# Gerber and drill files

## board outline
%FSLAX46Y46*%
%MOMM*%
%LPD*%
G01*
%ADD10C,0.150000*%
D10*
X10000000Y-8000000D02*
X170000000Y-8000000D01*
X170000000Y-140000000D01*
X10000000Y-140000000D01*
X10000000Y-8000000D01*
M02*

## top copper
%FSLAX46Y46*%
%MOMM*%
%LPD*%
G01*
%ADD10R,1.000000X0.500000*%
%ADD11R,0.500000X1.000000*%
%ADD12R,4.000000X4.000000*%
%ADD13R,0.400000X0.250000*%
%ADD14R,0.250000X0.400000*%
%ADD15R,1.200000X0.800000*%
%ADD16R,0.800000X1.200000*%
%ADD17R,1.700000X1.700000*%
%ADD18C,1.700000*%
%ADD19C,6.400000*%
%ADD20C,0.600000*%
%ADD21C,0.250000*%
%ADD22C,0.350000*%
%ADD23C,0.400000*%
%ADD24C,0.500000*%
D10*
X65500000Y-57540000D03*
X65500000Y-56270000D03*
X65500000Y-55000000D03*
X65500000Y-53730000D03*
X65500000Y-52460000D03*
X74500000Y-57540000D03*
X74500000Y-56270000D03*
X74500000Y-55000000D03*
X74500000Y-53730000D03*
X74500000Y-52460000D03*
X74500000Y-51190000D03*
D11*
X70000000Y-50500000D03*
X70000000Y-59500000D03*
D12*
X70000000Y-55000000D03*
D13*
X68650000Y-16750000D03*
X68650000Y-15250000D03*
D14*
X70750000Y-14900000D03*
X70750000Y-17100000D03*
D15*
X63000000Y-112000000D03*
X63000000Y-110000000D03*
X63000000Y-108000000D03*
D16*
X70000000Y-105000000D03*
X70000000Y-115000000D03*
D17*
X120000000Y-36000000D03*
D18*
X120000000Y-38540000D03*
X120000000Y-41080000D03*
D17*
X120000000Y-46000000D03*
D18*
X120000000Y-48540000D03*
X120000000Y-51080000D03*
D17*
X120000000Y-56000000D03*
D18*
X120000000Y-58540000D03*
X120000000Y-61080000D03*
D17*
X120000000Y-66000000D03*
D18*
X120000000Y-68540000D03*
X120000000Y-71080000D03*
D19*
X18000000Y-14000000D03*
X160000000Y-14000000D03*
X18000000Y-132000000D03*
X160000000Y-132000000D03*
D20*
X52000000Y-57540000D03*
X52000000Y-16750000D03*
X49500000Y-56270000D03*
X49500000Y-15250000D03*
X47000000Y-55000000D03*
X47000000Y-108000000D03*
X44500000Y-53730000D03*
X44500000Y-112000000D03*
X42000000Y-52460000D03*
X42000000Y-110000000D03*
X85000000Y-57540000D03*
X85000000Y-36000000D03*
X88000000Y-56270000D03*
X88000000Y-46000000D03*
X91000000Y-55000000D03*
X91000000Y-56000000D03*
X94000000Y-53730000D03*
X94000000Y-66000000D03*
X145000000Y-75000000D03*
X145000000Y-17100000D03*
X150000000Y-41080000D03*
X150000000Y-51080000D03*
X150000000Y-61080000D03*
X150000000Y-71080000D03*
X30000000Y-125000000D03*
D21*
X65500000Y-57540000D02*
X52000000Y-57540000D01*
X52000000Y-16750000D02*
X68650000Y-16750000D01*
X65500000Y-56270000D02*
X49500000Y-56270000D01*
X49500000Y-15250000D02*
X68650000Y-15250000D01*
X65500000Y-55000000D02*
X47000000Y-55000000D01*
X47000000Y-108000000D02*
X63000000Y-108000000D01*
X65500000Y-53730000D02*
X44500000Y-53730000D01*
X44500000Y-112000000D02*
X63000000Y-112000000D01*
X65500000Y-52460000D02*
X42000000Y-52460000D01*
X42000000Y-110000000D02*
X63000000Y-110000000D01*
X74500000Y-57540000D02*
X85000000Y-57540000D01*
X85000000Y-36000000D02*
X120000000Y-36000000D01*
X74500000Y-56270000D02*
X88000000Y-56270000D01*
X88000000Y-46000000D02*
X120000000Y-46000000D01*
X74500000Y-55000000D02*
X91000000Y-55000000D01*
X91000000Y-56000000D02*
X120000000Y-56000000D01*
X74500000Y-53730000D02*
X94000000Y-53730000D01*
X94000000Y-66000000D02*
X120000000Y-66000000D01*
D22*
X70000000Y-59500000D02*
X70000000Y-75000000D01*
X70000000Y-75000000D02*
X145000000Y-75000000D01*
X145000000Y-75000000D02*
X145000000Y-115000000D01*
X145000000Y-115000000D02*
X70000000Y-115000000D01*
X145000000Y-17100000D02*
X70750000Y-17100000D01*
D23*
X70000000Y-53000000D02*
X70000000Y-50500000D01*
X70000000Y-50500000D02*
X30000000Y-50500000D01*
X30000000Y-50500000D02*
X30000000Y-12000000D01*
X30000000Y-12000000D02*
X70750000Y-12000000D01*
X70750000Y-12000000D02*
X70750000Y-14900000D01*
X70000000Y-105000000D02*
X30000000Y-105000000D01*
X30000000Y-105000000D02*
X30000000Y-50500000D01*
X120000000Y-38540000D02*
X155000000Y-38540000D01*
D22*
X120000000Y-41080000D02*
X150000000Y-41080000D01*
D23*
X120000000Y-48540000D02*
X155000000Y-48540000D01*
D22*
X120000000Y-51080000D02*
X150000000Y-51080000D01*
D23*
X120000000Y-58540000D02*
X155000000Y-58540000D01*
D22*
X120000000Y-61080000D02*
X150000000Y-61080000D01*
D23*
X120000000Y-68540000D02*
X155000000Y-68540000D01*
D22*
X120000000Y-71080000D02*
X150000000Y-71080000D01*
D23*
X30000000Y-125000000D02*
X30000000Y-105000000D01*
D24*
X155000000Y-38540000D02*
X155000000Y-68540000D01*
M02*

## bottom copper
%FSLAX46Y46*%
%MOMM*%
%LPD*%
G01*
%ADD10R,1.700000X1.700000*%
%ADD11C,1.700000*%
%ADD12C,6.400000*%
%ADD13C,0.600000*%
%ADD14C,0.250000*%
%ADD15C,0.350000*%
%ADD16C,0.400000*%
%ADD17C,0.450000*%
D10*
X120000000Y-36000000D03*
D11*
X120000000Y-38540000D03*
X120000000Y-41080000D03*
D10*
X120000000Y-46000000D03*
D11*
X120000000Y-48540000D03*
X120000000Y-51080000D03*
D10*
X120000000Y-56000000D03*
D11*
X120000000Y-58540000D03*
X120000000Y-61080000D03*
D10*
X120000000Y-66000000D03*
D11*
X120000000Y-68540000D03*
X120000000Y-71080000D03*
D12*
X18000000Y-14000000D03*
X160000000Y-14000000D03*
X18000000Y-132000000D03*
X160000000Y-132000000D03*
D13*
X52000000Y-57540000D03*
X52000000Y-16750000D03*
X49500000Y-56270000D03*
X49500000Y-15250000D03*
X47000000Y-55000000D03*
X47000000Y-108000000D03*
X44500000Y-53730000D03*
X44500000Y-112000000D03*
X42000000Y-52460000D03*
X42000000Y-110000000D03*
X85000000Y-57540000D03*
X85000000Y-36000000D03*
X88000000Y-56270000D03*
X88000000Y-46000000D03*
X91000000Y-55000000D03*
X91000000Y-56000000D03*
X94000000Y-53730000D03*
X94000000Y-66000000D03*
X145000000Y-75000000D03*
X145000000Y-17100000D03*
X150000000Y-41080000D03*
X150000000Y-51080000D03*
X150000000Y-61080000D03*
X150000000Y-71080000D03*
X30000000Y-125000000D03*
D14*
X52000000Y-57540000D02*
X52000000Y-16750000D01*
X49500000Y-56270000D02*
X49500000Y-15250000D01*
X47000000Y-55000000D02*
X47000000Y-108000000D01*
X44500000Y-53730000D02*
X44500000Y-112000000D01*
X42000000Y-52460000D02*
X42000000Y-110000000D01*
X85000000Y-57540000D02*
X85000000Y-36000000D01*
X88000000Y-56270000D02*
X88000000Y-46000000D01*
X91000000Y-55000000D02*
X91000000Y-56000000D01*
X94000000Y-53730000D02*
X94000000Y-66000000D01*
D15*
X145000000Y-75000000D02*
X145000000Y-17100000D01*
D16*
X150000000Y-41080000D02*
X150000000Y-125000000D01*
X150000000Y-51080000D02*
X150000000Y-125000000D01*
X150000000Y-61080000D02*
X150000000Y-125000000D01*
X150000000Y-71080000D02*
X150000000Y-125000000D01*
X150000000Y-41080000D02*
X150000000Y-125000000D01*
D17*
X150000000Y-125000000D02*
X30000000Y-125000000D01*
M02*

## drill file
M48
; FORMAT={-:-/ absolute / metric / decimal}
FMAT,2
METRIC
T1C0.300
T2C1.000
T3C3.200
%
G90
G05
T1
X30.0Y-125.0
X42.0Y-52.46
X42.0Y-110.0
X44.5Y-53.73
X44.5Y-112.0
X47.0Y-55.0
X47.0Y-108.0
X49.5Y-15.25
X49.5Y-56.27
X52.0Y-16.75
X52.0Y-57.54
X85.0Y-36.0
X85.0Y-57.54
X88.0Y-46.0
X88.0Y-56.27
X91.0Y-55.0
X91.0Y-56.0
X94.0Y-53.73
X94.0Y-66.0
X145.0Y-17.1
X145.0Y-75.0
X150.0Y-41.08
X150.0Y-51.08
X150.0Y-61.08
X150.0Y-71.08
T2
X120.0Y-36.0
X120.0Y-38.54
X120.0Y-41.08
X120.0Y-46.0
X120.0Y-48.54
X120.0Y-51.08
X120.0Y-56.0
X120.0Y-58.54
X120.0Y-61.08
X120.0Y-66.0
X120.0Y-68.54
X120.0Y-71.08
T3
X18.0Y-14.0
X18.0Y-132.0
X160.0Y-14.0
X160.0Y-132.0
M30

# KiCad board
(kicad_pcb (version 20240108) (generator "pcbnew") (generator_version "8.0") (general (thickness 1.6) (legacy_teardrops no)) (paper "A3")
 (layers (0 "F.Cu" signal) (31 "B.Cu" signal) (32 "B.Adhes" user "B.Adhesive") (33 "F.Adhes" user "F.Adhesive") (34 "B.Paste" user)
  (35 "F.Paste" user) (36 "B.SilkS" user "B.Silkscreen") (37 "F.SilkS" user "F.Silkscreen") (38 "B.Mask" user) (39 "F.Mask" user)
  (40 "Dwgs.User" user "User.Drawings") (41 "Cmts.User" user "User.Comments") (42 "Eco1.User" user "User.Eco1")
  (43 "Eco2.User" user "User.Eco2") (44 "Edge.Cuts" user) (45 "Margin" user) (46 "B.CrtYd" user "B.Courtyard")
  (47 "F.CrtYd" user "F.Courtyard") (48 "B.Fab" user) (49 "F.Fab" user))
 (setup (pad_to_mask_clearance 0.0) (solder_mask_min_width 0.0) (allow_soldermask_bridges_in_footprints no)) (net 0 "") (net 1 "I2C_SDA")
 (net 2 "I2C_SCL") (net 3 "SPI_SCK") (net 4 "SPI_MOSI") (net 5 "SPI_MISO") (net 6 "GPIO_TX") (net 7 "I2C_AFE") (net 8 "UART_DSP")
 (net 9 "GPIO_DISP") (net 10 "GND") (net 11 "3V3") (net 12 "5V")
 (gr_rect (start 10 8) (end 170 140) (stroke (width 0.15) (type solid)) (fill none) (layer "Edge.Cuts"))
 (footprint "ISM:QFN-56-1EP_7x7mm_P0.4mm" (layer "F.Cu") (at 70 55)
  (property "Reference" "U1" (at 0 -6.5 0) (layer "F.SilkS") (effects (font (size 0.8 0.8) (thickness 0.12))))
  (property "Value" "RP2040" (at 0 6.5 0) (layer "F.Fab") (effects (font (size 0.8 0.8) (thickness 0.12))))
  (pad "1" smd rect (at -4.5 2.54) (size 1.0 0.5) (layers "F.Cu" "F.Paste" "F.Mask") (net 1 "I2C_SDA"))
  (pad "2" smd rect (at -4.5 1.27) (size 1.0 0.5) (layers "F.Cu" "F.Paste" "F.Mask") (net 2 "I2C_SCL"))
  (pad "3" smd rect (at -4.5 0) (size 1.0 0.5) (layers "F.Cu" "F.Paste" "F.Mask") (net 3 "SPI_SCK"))
  (pad "4" smd rect (at -4.5 -1.27) (size 1.0 0.5) (layers "F.Cu" "F.Paste" "F.Mask") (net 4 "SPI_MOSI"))
  (pad "5" smd rect (at -4.5 -2.54) (size 1.0 0.5) (layers "F.Cu" "F.Paste" "F.Mask") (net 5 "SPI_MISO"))
  (pad "6" smd rect (at 4.5 2.54) (size 1.0 0.5) (layers "F.Cu" "F.Paste" "F.Mask") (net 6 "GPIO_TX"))
  (pad "7" smd rect (at 4.5 1.27) (size 1.0 0.5) (layers "F.Cu" "F.Paste" "F.Mask") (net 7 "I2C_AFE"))
  (pad "8" smd rect (at 4.5 0) (size 1.0 0.5) (layers "F.Cu" "F.Paste" "F.Mask") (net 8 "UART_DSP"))
  (pad "9" smd rect (at 4.5 -1.27) (size 1.0 0.5) (layers "F.Cu" "F.Paste" "F.Mask") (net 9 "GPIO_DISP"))
  (pad "12" smd rect (at 4.5 -2.54) (size 1.0 0.5) (layers "F.Cu" "F.Paste" "F.Mask"))
  (pad "13" smd rect (at 4.5 -3.81) (size 1.0 0.5) (layers "F.Cu" "F.Paste" "F.Mask"))
  (pad "10" smd rect (at 0 -4.5) (size 0.5 1.0) (layers "F.Cu" "F.Paste" "F.Mask") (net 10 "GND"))
  (pad "11" smd rect (at 0 4.5) (size 0.5 1.0) (layers "F.Cu" "F.Paste" "F.Mask") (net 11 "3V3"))
  (pad "EP" smd rect (at 0 0) (size 4 4) (layers "F.Cu" "F.Paste" "F.Mask") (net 10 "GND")))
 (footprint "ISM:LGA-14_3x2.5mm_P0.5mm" (layer "F.Cu") (at 70 16)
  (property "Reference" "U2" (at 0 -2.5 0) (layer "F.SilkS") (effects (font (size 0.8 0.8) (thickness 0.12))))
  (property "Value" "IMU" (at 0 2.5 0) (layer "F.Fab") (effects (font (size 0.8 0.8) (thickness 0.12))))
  (pad "1" smd rect (at -1.35 0.75) (size 0.4 0.25) (layers "F.Cu" "F.Paste" "F.Mask") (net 1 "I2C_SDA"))
  (pad "2" smd rect (at -1.35 -0.75) (size 0.4 0.25) (layers "F.Cu" "F.Paste" "F.Mask") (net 2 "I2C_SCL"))
  (pad "3" smd rect (at 0.75 -1.1) (size 0.25 0.4) (layers "F.Cu" "F.Paste" "F.Mask") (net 10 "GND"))
  (pad "4" smd rect (at 0.75 1.1) (size 0.25 0.4) (layers "F.Cu" "F.Paste" "F.Mask") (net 11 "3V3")))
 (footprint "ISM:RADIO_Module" (layer "F.Cu") (at 70 110)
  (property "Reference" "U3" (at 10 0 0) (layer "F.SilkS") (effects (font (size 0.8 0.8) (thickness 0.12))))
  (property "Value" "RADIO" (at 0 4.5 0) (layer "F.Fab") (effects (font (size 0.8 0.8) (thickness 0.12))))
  (pad "1" smd rect (at -7 2) (size 1.2 0.8) (layers "F.Cu" "F.Paste" "F.Mask") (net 4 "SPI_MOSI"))
  (pad "2" smd rect (at -7 0) (size 1.2 0.8) (layers "F.Cu" "F.Paste" "F.Mask") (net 5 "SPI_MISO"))
  (pad "3" smd rect (at -7 -2) (size 1.2 0.8) (layers "F.Cu" "F.Paste" "F.Mask") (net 3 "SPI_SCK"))
  (pad "4" smd rect (at 0 -5) (size 0.8 1.2) (layers "F.Cu" "F.Paste" "F.Mask") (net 10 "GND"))
  (pad "5" smd rect (at 0 5) (size 0.8 1.2) (layers "F.Cu" "F.Paste" "F.Mask") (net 11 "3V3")))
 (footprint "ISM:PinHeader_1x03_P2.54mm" (layer "F.Cu") (at 120 36)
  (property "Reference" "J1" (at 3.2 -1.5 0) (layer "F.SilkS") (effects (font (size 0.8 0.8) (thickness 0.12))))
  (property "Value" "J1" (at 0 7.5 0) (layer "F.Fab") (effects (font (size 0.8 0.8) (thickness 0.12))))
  (pad "1" thru_hole rect (at 0 0) (size 1.7 1.7) (drill 1.0) (layers "*.Cu" "*.Mask") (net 6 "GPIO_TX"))
  (pad "2" thru_hole circle (at 0 2.54) (size 1.7 1.7) (drill 1.0) (layers "*.Cu" "*.Mask") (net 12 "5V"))
  (pad "3" thru_hole circle (at 0 5.08) (size 1.7 1.7) (drill 1.0) (layers "*.Cu" "*.Mask") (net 10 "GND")))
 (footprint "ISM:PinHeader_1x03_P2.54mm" (layer "F.Cu") (at 120 46)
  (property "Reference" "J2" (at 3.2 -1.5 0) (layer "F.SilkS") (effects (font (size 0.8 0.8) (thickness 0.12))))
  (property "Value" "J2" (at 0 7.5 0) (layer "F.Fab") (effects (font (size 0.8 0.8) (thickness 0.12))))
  (pad "1" thru_hole rect (at 0 0) (size 1.7 1.7) (drill 1.0) (layers "*.Cu" "*.Mask") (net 7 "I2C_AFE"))
  (pad "2" thru_hole circle (at 0 2.54) (size 1.7 1.7) (drill 1.0) (layers "*.Cu" "*.Mask") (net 12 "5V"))
  (pad "3" thru_hole circle (at 0 5.08) (size 1.7 1.7) (drill 1.0) (layers "*.Cu" "*.Mask") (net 10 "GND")))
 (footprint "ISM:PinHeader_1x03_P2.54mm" (layer "F.Cu") (at 120 56)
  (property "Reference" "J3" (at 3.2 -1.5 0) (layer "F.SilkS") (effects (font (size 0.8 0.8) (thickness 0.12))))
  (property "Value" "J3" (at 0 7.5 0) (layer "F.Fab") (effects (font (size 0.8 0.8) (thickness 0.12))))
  (pad "1" thru_hole rect (at 0 0) (size 1.7 1.7) (drill 1.0) (layers "*.Cu" "*.Mask") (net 8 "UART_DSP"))
  (pad "2" thru_hole circle (at 0 2.54) (size 1.7 1.7) (drill 1.0) (layers "*.Cu" "*.Mask") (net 12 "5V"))
  (pad "3" thru_hole circle (at 0 5.08) (size 1.7 1.7) (drill 1.0) (layers "*.Cu" "*.Mask") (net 10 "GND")))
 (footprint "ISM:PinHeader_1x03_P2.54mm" (layer "F.Cu") (at 120 66)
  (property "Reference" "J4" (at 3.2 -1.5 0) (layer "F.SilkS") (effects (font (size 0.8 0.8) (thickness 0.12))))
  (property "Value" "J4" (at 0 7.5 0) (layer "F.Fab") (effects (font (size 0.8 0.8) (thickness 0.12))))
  (pad "1" thru_hole rect (at 0 0) (size 1.7 1.7) (drill 1.0) (layers "*.Cu" "*.Mask") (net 9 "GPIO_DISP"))
  (pad "2" thru_hole circle (at 0 2.54) (size 1.7 1.7) (drill 1.0) (layers "*.Cu" "*.Mask") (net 12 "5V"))
  (pad "3" thru_hole circle (at 0 5.08) (size 1.7 1.7) (drill 1.0) (layers "*.Cu" "*.Mask") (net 10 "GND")))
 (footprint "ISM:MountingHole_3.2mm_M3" (layer "F.Cu") (at 18 14)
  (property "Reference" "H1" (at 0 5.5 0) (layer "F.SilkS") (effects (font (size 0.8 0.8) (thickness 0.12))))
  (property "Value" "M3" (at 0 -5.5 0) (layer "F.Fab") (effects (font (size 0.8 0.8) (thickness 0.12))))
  (pad "" thru_hole circle (at 0 0) (size 6.4 6.4) (drill 3.2) (layers "*.Cu" "*.Mask")))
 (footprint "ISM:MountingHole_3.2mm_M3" (layer "F.Cu") (at 160 14)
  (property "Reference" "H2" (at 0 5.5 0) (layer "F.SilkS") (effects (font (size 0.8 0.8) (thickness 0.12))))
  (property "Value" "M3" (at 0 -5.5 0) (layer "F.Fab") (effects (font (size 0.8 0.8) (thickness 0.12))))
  (pad "" thru_hole circle (at 0 0) (size 6.4 6.4) (drill 3.2) (layers "*.Cu" "*.Mask")))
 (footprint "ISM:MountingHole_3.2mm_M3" (layer "F.Cu") (at 18 132)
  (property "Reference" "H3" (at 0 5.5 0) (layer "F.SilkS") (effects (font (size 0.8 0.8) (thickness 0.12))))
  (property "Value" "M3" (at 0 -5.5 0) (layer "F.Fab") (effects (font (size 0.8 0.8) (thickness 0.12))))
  (pad "" thru_hole circle (at 0 0) (size 6.4 6.4) (drill 3.2) (layers "*.Cu" "*.Mask")))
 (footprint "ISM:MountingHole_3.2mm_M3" (layer "F.Cu") (at 160 132)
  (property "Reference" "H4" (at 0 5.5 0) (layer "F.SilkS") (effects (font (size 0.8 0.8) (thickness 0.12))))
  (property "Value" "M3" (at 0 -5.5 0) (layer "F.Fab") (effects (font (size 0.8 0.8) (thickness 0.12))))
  (pad "" thru_hole circle (at 0 0) (size 6.4 6.4) (drill 3.2) (layers "*.Cu" "*.Mask")))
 (segment (start 65.5 57.54) (end 52.0 57.54) (width 0.25) (layer "F.Cu") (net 1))
 (segment (start 52.0 57.54) (end 52.0 16.75) (width 0.25) (layer "B.Cu") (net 1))
 (segment (start 52.0 16.75) (end 68.65 16.75) (width 0.25) (layer "F.Cu") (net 1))
 (segment (start 65.5 56.27) (end 49.5 56.27) (width 0.25) (layer "F.Cu") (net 2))
 (segment (start 49.5 56.27) (end 49.5 15.25) (width 0.25) (layer "B.Cu") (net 2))
 (segment (start 49.5 15.25) (end 68.65 15.25) (width 0.25) (layer "F.Cu") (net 2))
 (segment (start 65.5 55) (end 47.0 55) (width 0.25) (layer "F.Cu") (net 3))
 (segment (start 47.0 55) (end 47.0 108) (width 0.25) (layer "B.Cu") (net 3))
 (segment (start 47.0 108) (end 63 108) (width 0.25) (layer "F.Cu") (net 3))
 (segment (start 65.5 53.73) (end 44.5 53.73) (width 0.25) (layer "F.Cu") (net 4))
 (segment (start 44.5 53.73) (end 44.5 112) (width 0.25) (layer "B.Cu") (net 4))
 (segment (start 44.5 112) (end 63 112) (width 0.25) (layer "F.Cu") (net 4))
 (segment (start 65.5 52.46) (end 42.0 52.46) (width 0.25) (layer "F.Cu") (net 5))
 (segment (start 42.0 52.46) (end 42.0 110) (width 0.25) (layer "B.Cu") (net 5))
 (segment (start 42.0 110) (end 63 110) (width 0.25) (layer "F.Cu") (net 5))
 (segment (start 74.5 57.54) (end 85 57.54) (width 0.25) (layer "F.Cu") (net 6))
 (segment (start 85 57.54) (end 85 36) (width 0.25) (layer "B.Cu") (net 6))
 (segment (start 85 36) (end 120 36) (width 0.25) (layer "F.Cu") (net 6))
 (segment (start 74.5 56.27) (end 88 56.27) (width 0.25) (layer "F.Cu") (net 7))
 (segment (start 88 56.27) (end 88 46) (width 0.25) (layer "B.Cu") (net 7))
 (segment (start 88 46) (end 120 46) (width 0.25) (layer "F.Cu") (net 7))
 (segment (start 74.5 55) (end 91 55) (width 0.25) (layer "F.Cu") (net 8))
 (segment (start 91 55) (end 91 56) (width 0.25) (layer "B.Cu") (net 8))
 (segment (start 91 56) (end 120 56) (width 0.25) (layer "F.Cu") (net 8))
 (segment (start 74.5 53.73) (end 94 53.73) (width 0.25) (layer "F.Cu") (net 9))
 (segment (start 94 53.73) (end 94 66) (width 0.25) (layer "B.Cu") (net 9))
 (segment (start 94 66) (end 120 66) (width 0.25) (layer "F.Cu") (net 9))
 (segment (start 70 59.5) (end 70 75) (width 0.35) (layer "F.Cu") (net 11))
 (segment (start 70 75) (end 145 75) (width 0.35) (layer "F.Cu") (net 11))
 (segment (start 145 75) (end 145 115) (width 0.35) (layer "F.Cu") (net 11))
 (segment (start 145 115) (end 70 115) (width 0.35) (layer "F.Cu") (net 11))
 (segment (start 145 75) (end 145 17.1) (width 0.35) (layer "B.Cu") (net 11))
 (segment (start 145 17.1) (end 70.75 17.1) (width 0.35) (layer "F.Cu") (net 11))
 (segment (start 70 53) (end 70 50.5) (width 0.4) (layer "F.Cu") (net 10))
 (segment (start 70 50.5) (end 30 50.5) (width 0.4) (layer "F.Cu") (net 10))
 (segment (start 30 50.5) (end 30 12) (width 0.4) (layer "F.Cu") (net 10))
 (segment (start 30 12) (end 70.75 12) (width 0.4) (layer "F.Cu") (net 10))
 (segment (start 70.75 12) (end 70.75 14.9) (width 0.4) (layer "F.Cu") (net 10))
 (segment (start 70 105) (end 30 105) (width 0.4) (layer "F.Cu") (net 10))
 (segment (start 30 105) (end 30 50.5) (width 0.4) (layer "F.Cu") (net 10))
 (segment (start 120 38.54) (end 155 38.54) (width 0.4) (layer "F.Cu") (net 12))
 (segment (start 120 41.08) (end 150 41.08) (width 0.35) (layer "F.Cu") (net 10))
 (segment (start 150 41.08) (end 150 125) (width 0.4) (layer "B.Cu") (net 10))
 (segment (start 120 48.54) (end 155 48.54) (width 0.4) (layer "F.Cu") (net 12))
 (segment (start 120 51.08) (end 150 51.08) (width 0.35) (layer "F.Cu") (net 10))
 (segment (start 150 51.08) (end 150 125) (width 0.4) (layer "B.Cu") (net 10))
 (segment (start 120 58.54) (end 155 58.54) (width 0.4) (layer "F.Cu") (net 12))
 (segment (start 120 61.08) (end 150 61.08) (width 0.35) (layer "F.Cu") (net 10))
 (segment (start 150 61.08) (end 150 125) (width 0.4) (layer "B.Cu") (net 10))
 (segment (start 120 68.54) (end 155 68.54) (width 0.4) (layer "F.Cu") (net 12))
 (segment (start 120 71.08) (end 150 71.08) (width 0.35) (layer "F.Cu") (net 10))
 (segment (start 150 71.08) (end 150 125) (width 0.4) (layer "B.Cu") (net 10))
 (segment (start 150 41.08) (end 150 125) (width 0.4) (layer "B.Cu") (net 10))
 (segment (start 150 125) (end 30 125) (width 0.45) (layer "B.Cu") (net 10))
 (segment (start 30 125) (end 30 105) (width 0.4) (layer "F.Cu") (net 10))
 (segment (start 155 38.54) (end 155 68.54) (width 0.5) (layer "F.Cu") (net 12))
 (via (at 52.0 57.54) (size 0.6) (drill 0.3) (layers "F.Cu" "B.Cu") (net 1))
 (via (at 52.0 16.75) (size 0.6) (drill 0.3) (layers "F.Cu" "B.Cu") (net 1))
 (via (at 49.5 56.27) (size 0.6) (drill 0.3) (layers "F.Cu" "B.Cu") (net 2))
 (via (at 49.5 15.25) (size 0.6) (drill 0.3) (layers "F.Cu" "B.Cu") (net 2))
 (via (at 47.0 55) (size 0.6) (drill 0.3) (layers "F.Cu" "B.Cu") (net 3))
 (via (at 47.0 108) (size 0.6) (drill 0.3) (layers "F.Cu" "B.Cu") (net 3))
 (via (at 44.5 53.73) (size 0.6) (drill 0.3) (layers "F.Cu" "B.Cu") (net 4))
 (via (at 44.5 112) (size 0.6) (drill 0.3) (layers "F.Cu" "B.Cu") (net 4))
 (via (at 42.0 52.46) (size 0.6) (drill 0.3) (layers "F.Cu" "B.Cu") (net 5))
 (via (at 42.0 110) (size 0.6) (drill 0.3) (layers "F.Cu" "B.Cu") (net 5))
 (via (at 85 57.54) (size 0.6) (drill 0.3) (layers "F.Cu" "B.Cu") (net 6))
 (via (at 85 36) (size 0.6) (drill 0.3) (layers "F.Cu" "B.Cu") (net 6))
 (via (at 88 56.27) (size 0.6) (drill 0.3) (layers "F.Cu" "B.Cu") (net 7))
 (via (at 88 46) (size 0.6) (drill 0.3) (layers "F.Cu" "B.Cu") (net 7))
 (via (at 91 55) (size 0.6) (drill 0.3) (layers "F.Cu" "B.Cu") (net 8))
 (via (at 91 56) (size 0.6) (drill 0.3) (layers "F.Cu" "B.Cu") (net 8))
 (via (at 94 53.73) (size 0.6) (drill 0.3) (layers "F.Cu" "B.Cu") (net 9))
 (via (at 94 66) (size 0.6) (drill 0.3) (layers "F.Cu" "B.Cu") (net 9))
 (via (at 145 75) (size 0.6) (drill 0.3) (layers "F.Cu" "B.Cu") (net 11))
 (via (at 145 17.1) (size 0.6) (drill 0.3) (layers "F.Cu" "B.Cu") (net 11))
 (via (at 150 41.08) (size 0.6) (drill 0.3) (layers "F.Cu" "B.Cu") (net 10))
 (via (at 150 51.08) (size 0.6) (drill 0.3) (layers "F.Cu" "B.Cu") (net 10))
 (via (at 150 61.08) (size 0.6) (drill 0.3) (layers "F.Cu" "B.Cu") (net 10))
 (via (at 150 71.08) (size 0.6) (drill 0.3) (layers "F.Cu" "B.Cu") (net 10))
 (via (at 30 125) (size 0.6) (drill 0.3) (layers "F.Cu" "B.Cu") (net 10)))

